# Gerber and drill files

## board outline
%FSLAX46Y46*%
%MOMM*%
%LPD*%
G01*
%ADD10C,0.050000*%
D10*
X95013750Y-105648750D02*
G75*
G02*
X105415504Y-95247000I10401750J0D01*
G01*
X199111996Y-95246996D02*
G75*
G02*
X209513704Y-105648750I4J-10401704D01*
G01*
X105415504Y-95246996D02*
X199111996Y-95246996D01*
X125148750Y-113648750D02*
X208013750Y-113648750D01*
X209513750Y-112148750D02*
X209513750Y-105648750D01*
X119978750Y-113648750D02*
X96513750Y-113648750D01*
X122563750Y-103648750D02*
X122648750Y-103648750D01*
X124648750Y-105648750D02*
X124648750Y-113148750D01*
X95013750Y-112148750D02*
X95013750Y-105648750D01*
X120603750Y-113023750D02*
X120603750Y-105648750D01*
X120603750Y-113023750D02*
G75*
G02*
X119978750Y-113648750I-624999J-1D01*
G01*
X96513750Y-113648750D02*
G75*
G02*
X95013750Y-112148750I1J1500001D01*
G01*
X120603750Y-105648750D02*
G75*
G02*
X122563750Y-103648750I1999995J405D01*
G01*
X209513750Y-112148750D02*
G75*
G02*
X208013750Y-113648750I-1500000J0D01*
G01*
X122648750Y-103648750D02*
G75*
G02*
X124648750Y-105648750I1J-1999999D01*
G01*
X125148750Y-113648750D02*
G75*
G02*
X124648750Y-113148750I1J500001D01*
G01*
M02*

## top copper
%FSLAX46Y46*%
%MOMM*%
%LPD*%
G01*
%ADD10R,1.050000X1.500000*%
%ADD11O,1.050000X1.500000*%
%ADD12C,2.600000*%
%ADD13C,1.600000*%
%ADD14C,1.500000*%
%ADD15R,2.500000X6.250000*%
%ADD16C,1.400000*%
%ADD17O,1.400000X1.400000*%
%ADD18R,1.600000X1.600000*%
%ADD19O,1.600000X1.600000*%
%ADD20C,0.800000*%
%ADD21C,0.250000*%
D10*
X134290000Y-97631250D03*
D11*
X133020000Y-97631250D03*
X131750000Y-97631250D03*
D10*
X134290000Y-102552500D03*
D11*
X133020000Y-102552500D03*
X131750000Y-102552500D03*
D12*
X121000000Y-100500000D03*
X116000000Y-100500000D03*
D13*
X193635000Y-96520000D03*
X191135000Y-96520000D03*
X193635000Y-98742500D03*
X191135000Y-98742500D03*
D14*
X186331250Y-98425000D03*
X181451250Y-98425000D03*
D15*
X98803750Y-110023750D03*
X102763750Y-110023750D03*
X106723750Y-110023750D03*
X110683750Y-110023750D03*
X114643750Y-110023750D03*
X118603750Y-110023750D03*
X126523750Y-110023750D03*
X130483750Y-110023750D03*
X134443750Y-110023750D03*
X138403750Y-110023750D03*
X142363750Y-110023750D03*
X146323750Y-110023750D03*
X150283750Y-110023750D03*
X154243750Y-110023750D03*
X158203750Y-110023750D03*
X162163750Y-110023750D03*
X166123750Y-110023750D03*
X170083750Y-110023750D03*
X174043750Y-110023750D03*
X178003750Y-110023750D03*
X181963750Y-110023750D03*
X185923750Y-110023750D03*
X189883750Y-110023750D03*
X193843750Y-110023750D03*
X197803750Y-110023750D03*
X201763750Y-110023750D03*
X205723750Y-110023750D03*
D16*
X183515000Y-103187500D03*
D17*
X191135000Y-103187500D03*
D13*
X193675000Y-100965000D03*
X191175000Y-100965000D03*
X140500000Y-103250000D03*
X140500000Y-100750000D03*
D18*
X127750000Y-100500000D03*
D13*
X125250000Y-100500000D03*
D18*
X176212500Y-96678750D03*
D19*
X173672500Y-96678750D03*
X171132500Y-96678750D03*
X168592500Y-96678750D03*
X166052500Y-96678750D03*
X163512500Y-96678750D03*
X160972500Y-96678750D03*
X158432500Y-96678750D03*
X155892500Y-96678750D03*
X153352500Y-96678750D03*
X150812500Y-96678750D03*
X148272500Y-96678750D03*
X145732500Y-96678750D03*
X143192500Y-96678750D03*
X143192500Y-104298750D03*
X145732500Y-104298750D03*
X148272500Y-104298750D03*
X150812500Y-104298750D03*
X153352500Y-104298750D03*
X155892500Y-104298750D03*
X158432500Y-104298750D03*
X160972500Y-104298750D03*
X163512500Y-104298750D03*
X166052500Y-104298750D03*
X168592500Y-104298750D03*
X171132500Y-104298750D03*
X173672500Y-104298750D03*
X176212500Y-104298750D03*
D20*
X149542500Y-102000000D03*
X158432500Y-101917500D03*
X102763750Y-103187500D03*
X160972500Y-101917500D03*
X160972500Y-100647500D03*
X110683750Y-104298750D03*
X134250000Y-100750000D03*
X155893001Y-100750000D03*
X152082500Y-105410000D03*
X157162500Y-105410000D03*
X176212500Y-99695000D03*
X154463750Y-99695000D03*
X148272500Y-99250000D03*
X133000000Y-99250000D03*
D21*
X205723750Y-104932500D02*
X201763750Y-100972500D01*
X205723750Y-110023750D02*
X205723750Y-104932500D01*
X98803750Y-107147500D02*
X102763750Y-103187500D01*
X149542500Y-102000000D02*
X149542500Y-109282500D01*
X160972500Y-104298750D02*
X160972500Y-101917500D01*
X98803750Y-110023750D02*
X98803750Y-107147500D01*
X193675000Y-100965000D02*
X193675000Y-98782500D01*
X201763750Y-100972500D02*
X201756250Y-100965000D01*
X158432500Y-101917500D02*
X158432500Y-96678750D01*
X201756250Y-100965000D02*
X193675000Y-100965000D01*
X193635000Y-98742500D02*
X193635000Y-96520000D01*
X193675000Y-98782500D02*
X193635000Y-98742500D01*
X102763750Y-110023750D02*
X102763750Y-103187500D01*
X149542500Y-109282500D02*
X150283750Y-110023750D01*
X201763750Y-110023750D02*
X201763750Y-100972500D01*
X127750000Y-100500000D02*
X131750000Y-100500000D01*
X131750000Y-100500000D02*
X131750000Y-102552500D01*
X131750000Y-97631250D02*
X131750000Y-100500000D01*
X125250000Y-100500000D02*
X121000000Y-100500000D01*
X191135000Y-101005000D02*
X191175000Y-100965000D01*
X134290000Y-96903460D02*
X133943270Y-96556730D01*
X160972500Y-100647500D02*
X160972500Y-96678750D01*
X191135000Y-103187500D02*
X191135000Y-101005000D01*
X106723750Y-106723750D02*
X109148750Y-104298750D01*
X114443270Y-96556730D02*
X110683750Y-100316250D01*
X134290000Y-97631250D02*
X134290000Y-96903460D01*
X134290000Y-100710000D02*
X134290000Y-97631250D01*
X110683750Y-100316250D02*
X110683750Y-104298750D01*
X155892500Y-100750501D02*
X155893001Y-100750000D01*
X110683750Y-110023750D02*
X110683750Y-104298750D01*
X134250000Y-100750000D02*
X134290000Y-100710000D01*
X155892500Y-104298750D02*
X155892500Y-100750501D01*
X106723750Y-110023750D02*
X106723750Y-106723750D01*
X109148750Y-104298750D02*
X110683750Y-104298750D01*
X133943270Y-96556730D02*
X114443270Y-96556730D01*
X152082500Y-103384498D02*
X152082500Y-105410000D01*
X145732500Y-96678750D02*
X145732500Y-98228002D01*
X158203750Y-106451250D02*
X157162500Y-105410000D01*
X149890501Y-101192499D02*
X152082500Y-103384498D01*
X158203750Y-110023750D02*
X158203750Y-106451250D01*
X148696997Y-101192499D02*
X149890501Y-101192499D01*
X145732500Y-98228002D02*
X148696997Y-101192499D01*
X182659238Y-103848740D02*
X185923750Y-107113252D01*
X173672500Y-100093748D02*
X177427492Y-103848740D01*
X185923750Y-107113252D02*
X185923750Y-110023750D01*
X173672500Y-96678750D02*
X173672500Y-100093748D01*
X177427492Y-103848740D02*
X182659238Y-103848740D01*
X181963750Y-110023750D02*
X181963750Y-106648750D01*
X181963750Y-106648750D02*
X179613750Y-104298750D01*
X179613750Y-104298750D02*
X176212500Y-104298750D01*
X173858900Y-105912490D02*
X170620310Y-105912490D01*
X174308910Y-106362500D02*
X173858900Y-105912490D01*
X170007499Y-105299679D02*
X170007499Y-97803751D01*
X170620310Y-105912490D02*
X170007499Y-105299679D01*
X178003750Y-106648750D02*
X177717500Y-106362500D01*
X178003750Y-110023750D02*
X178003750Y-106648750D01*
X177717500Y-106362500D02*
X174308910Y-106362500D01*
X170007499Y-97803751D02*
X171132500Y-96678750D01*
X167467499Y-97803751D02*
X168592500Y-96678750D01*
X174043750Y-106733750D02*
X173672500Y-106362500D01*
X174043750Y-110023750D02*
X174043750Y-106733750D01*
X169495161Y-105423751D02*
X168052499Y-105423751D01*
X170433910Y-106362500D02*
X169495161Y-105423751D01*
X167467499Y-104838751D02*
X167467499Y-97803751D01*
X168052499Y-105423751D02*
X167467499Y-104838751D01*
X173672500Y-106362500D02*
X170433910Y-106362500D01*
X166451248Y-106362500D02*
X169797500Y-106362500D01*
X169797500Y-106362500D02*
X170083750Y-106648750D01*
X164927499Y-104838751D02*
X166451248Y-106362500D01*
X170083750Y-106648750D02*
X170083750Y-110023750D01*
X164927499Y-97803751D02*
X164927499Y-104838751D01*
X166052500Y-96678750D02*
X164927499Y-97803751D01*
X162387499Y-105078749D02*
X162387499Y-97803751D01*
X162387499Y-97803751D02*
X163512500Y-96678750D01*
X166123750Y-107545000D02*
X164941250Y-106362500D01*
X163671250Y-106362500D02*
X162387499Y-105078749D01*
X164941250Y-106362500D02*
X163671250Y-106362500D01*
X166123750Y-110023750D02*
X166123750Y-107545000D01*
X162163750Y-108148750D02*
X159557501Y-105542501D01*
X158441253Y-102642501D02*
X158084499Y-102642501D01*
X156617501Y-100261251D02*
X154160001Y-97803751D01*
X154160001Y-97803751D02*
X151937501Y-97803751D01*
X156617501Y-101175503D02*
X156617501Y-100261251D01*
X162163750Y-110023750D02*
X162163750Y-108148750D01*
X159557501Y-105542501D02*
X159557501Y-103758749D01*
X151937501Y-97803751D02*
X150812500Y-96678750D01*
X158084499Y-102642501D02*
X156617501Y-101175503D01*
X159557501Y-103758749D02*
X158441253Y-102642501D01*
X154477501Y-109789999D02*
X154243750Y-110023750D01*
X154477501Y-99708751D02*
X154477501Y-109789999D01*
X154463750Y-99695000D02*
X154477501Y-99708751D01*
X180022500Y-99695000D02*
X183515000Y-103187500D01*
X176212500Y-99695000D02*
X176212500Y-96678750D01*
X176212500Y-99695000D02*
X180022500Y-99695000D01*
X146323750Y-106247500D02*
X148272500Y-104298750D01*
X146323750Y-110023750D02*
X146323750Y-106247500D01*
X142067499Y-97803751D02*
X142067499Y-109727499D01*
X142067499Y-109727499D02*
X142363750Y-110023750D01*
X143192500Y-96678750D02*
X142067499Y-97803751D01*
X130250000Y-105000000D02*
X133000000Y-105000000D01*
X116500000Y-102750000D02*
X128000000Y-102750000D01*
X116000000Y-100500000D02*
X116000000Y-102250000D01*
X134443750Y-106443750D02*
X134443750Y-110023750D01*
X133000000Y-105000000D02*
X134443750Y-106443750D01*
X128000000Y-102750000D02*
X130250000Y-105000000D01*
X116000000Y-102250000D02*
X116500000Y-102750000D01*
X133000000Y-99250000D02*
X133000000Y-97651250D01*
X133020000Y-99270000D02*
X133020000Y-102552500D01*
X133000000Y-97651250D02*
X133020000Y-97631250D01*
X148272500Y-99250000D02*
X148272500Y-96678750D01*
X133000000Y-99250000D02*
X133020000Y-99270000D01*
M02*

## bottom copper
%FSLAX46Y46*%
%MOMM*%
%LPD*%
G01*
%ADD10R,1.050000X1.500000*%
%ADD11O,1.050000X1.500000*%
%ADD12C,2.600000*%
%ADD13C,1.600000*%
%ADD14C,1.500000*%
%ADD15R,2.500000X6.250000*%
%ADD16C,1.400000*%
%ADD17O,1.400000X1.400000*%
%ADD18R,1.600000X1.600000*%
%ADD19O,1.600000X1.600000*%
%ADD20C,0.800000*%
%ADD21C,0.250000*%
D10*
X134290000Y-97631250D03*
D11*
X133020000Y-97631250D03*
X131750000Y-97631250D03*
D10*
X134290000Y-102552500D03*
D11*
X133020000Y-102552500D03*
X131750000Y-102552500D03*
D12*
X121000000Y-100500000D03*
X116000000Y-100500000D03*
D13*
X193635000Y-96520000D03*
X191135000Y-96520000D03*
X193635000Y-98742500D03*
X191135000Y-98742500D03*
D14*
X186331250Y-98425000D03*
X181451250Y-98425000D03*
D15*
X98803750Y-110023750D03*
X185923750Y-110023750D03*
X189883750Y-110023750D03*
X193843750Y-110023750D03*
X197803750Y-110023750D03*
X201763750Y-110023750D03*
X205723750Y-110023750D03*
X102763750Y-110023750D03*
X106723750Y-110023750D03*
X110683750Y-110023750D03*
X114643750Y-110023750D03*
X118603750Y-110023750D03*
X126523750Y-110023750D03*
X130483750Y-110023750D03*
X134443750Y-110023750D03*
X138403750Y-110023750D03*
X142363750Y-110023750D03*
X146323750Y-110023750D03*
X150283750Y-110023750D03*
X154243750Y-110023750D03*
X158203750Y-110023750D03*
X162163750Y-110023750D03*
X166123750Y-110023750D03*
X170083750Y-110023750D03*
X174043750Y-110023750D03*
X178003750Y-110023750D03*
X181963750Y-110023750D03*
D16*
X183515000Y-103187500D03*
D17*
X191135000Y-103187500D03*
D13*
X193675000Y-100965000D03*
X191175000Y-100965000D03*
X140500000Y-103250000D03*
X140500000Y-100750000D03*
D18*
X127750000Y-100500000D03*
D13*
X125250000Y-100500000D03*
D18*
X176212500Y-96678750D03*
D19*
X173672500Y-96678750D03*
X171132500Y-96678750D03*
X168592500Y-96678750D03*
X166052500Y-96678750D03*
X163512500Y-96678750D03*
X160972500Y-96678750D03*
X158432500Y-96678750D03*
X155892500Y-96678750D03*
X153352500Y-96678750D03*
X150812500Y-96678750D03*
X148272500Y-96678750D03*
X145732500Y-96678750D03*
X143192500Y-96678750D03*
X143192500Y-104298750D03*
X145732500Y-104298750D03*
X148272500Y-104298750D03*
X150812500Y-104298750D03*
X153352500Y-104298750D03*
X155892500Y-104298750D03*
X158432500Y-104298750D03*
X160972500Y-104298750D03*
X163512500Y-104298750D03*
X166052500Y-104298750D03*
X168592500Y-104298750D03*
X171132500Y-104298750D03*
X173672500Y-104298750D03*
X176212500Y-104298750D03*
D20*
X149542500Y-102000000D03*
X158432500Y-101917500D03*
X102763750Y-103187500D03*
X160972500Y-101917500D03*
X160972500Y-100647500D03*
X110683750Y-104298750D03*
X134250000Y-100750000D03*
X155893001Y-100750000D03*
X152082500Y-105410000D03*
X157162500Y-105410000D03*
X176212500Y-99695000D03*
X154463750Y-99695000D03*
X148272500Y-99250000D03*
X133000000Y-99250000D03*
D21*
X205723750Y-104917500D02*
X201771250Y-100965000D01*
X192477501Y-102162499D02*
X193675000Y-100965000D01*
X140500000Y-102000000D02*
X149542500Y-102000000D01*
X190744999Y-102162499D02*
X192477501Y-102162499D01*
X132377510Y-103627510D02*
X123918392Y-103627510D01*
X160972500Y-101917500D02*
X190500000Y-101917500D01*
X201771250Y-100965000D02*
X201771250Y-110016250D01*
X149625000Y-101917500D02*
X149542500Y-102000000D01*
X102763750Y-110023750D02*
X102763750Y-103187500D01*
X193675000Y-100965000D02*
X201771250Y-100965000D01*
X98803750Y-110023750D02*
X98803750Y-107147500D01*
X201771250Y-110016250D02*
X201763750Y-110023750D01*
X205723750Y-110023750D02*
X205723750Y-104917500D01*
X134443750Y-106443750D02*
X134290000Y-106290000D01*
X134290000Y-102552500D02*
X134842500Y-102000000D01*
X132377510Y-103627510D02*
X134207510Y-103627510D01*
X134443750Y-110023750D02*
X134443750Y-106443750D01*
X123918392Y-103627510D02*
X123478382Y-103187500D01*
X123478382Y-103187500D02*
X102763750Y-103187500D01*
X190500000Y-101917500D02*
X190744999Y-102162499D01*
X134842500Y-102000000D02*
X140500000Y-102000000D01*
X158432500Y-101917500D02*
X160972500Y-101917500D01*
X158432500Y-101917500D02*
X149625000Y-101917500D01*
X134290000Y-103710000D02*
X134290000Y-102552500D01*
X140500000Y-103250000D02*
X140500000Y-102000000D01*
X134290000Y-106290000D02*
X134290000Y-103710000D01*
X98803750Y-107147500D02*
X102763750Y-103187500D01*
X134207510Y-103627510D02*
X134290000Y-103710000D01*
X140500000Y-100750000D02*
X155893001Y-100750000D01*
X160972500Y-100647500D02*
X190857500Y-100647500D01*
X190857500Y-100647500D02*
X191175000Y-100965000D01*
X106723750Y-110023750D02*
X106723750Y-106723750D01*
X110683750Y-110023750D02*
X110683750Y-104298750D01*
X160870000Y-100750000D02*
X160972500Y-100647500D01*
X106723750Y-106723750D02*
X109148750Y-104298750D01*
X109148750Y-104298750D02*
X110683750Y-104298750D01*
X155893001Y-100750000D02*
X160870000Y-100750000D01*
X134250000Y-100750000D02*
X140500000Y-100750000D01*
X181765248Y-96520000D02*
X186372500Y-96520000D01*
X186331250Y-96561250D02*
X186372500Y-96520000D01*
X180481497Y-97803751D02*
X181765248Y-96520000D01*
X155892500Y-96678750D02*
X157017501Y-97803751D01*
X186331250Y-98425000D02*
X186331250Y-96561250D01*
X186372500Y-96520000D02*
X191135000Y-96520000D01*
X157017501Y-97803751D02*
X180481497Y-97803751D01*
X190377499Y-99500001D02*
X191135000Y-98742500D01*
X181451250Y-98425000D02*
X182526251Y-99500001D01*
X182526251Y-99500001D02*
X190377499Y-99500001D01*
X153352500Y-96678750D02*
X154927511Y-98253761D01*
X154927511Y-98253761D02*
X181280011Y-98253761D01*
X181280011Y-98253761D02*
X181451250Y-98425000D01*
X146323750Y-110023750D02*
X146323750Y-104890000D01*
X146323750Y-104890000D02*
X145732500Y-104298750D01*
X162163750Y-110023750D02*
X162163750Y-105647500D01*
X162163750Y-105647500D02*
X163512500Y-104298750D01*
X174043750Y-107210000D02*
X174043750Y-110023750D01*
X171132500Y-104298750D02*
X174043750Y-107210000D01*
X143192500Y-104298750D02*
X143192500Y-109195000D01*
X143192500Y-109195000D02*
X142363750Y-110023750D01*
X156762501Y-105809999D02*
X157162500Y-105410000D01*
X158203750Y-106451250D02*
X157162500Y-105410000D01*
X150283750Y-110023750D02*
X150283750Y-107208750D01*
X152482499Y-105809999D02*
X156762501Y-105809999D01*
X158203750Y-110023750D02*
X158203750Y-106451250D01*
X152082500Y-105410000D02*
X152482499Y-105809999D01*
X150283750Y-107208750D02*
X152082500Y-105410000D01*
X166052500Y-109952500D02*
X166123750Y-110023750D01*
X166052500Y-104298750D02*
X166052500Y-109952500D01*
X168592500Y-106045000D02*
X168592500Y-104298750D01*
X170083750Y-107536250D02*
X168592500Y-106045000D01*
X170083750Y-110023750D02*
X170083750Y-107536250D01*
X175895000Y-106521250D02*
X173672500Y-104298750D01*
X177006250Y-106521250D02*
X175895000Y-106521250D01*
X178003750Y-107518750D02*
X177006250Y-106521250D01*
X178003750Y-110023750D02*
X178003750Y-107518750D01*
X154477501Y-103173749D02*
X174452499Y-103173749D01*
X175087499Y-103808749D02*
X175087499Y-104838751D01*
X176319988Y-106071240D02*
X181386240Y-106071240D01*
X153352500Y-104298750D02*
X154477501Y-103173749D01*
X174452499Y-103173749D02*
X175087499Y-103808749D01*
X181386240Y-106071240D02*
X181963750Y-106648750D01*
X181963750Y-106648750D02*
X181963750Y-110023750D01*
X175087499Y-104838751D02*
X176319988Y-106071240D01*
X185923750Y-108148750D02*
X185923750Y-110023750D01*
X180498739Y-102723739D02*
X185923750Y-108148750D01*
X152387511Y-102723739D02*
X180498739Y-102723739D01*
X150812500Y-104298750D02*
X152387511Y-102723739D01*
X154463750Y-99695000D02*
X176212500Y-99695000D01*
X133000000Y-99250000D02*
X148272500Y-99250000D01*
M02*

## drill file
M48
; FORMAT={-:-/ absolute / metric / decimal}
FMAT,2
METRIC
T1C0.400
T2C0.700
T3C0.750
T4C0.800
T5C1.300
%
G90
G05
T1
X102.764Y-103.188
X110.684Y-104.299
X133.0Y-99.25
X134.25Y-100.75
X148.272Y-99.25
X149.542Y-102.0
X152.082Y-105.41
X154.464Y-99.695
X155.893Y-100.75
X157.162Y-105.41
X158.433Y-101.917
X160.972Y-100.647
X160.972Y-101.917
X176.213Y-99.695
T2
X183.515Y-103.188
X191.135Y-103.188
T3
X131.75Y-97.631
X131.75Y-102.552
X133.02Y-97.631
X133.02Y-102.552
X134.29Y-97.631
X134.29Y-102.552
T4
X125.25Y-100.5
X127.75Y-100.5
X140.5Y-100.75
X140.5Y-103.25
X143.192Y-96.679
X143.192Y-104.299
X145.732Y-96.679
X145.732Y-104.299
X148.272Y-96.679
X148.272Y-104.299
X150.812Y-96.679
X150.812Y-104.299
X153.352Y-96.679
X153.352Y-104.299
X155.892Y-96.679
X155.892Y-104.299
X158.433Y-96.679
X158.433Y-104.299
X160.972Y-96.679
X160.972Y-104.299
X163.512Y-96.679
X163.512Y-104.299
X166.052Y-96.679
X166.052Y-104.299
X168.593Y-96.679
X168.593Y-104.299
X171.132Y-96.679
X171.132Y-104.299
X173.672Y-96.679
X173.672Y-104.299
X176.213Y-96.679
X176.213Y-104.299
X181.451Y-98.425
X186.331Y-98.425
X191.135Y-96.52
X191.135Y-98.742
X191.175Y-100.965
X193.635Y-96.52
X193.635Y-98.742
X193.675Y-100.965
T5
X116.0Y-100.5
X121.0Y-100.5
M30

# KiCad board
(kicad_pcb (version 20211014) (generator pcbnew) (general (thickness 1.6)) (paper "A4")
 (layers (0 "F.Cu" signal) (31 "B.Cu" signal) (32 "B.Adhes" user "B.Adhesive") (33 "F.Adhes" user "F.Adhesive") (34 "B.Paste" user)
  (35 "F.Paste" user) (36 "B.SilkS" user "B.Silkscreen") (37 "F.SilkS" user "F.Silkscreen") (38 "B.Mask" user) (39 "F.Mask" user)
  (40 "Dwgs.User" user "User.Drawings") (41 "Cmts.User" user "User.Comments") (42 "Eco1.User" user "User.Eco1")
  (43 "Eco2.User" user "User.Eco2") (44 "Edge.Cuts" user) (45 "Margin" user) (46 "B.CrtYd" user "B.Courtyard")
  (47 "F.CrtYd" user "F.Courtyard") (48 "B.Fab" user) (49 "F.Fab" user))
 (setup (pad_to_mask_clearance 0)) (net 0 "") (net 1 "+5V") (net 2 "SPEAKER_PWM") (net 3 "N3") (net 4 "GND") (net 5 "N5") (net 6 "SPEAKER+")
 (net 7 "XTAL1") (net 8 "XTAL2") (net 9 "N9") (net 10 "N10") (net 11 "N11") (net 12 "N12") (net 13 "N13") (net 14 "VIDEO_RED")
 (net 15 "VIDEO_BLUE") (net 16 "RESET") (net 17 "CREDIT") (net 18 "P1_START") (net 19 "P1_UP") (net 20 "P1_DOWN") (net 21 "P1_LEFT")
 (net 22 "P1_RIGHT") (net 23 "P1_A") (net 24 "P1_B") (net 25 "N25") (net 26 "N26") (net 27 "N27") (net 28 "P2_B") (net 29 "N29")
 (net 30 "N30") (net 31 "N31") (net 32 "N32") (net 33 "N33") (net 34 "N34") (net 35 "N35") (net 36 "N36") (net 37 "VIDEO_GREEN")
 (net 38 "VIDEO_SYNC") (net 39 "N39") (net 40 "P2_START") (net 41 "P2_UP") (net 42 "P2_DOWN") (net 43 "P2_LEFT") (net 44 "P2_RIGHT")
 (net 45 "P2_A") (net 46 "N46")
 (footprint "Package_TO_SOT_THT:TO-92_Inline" (layer "F.Cu") (at 134.29 97.63125 180)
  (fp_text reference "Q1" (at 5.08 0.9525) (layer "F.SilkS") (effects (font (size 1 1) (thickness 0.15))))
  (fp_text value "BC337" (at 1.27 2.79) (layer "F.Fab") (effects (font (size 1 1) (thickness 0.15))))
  (pad "1" thru_hole rect locked (at 0 0 180) (size 1.05 1.5) (drill 0.75) (layers *.Cu *.Mask) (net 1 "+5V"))
  (pad "2" thru_hole oval locked (at 1.27 0 180) (size 1.05 1.5) (drill 0.75) (layers *.Cu *.Mask) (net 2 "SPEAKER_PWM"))
  (pad "3" thru_hole oval locked (at 2.54 0 180) (size 1.05 1.5) (drill 0.75) (layers *.Cu *.Mask) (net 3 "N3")))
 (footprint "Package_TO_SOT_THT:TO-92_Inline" (layer "F.Cu") (at 134.29 102.5525 180)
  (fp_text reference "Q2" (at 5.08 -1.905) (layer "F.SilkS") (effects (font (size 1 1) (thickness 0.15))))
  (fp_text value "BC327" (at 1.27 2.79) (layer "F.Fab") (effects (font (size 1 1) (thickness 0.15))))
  (pad "1" thru_hole rect locked (at 0 0 180) (size 1.05 1.5) (drill 0.75) (layers *.Cu *.Mask) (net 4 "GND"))
  (pad "2" thru_hole oval locked (at 1.27 0 180) (size 1.05 1.5) (drill 0.75) (layers *.Cu *.Mask) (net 2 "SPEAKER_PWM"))
  (pad "3" thru_hole oval locked (at 2.54 0 180) (size 1.05 1.5) (drill 0.75) (layers *.Cu *.Mask) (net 3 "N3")))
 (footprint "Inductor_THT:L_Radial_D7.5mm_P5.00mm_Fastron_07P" (layer "F.Cu") (at 121 100.5 180)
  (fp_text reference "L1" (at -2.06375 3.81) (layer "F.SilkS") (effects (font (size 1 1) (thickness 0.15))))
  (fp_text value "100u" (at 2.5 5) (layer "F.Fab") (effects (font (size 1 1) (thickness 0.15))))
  (pad "1" thru_hole circle locked (at 0 0 180) (size 2.6 2.6) (drill 1.3) (layers *.Cu *.Mask) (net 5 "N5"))
  (pad "2" thru_hole circle locked (at 5 0 180) (size 2.6 2.6) (drill 1.3) (layers *.Cu *.Mask) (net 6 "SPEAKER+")))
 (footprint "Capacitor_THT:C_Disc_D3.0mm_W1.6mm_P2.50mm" (layer "F.Cu") (at 193.635 96.52 180)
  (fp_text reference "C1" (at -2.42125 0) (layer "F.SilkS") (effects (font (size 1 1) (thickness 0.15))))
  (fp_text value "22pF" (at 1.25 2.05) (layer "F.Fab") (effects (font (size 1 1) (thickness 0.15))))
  (pad "1" thru_hole circle locked (at 0 0 180) (size 1.6 1.6) (drill 0.8) (layers *.Cu *.Mask) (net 4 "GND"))
  (pad "2" thru_hole circle locked (at 2.5 0 180) (size 1.6 1.6) (drill 0.8) (layers *.Cu *.Mask) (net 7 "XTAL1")))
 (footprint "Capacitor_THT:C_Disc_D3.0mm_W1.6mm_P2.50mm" (layer "F.Cu") (at 193.635 98.7425 180)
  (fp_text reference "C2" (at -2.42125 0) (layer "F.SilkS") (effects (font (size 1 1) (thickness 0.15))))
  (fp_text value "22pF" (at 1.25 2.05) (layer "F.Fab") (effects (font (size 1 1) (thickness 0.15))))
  (pad "1" thru_hole circle locked (at 0 0 180) (size 1.6 1.6) (drill 0.8) (layers *.Cu *.Mask) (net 4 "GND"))
  (pad "2" thru_hole circle locked (at 2.5 0 180) (size 1.6 1.6) (drill 0.8) (layers *.Cu *.Mask) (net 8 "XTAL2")))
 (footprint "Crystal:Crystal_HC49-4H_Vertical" (layer "F.Cu") (at 186.33125 98.425 180)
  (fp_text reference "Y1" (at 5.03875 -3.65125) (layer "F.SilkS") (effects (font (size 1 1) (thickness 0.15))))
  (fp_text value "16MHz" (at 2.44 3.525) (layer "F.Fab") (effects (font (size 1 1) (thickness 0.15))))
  (pad "1" thru_hole circle locked (at 0 0 180) (size 1.5 1.5) (drill 0.8) (layers *.Cu *.Mask) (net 7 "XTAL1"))
  (pad "2" thru_hole circle locked (at 4.88 0 180) (size 1.5 1.5) (drill 0.8) (layers *.Cu *.Mask) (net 8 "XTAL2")))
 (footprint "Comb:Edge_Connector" (layer "F.Cu") (at 152.26375 105.64875)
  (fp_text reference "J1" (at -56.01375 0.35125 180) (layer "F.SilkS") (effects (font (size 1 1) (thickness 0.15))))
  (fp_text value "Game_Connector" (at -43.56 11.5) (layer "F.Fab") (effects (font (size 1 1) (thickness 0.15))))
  (fp_line (start -27.115 8) (end 55.75 8) (layer "Edge.Cuts") (width 0.05))
  (fp_line (start 57.25 6.5) (end 57.25 0) (layer "Edge.Cuts") (width 0.05))
  (fp_line (start -32.285 8) (end -55.75 8) (layer "Edge.Cuts") (width 0.05))
  (fp_line (start -29.7 -2) (end -29.615 -2) (layer "Edge.Cuts") (width 0.05))
  (fp_line (start -27.615 0) (end -27.615 7.5) (layer "Edge.Cuts") (width 0.05))
  (fp_line (start -57.25 6.5) (end -57.25 0) (layer "Edge.Cuts") (width 0.05))
  (fp_line (start -31.66 7.375) (end -31.66 0) (layer "Edge.Cuts") (width 0.05))
  (fp_arc (start -31.66 7.375) (mid -31.843058 7.816942) (end -32.285 8) (layer "Edge.Cuts") (width 0.05))
  (fp_arc (start -55.75 8) (mid -56.81066 7.56066) (end -57.25 6.5) (layer "Edge.Cuts") (width 0.05))
  (fp_arc (start -31.66 0) (mid -31.088427 -1.400259) (end -29.7 -2) (layer "Edge.Cuts") (width 0.05))
  (fp_arc (start 57.25 6.5) (mid 56.81066 7.56066) (end 55.75 8) (layer "Edge.Cuts") (width 0.05))
  (fp_arc (start -29.615 -2) (mid -28.200786 -1.414214) (end -27.615 0) (layer "Edge.Cuts") (width 0.05))
  (fp_arc (start -27.115 8) (mid -27.468553 7.853553) (end -27.615 7.5) (layer "Edge.Cuts") (width 0.05))
  (pad "1" smd rect (at -53.46 4.375) (size 2.5 6.25) (layers "F.Cu" "F.Paste" "F.Mask") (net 4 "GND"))
  (pad "2" smd rect (at -49.5 4.375) (size 2.5 6.25) (layers "F.Cu" "F.Paste" "F.Mask") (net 4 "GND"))
  (pad "3" smd rect (at -45.54 4.375) (size 2.5 6.25) (layers "F.Cu" "F.Paste" "F.Mask") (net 1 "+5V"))
  (pad "4" smd rect (at -41.58 4.375) (size 2.5 6.25) (layers "F.Cu" "F.Paste" "F.Mask") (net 1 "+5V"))
  (pad "5" smd rect (at -37.62 4.375) (size 2.5 6.25) (layers "F.Cu" "F.Paste" "F.Mask") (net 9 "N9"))
  (pad "6" smd rect (at -33.66 4.375) (size 2.5 6.25) (layers "F.Cu" "F.Paste" "F.Mask") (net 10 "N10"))
  (pad "8" smd rect (at -25.74 4.375) (size 2.5 6.25) (layers "F.Cu" "F.Paste" "F.Mask") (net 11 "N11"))
  (pad "9" smd rect (at -21.78 4.375) (size 2.5 6.25) (layers "F.Cu" "F.Paste" "F.Mask") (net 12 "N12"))
  (pad "10" smd rect (at -17.82 4.375) (size 2.5 6.25) (layers "F.Cu" "F.Paste" "F.Mask") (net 6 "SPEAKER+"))
  (pad "11" smd rect (at -13.86 4.375) (size 2.5 6.25) (layers "F.Cu" "F.Paste" "F.Mask") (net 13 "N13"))
  (pad "12" smd rect (at -9.9 4.375) (size 2.5 6.25) (layers "F.Cu" "F.Paste" "F.Mask") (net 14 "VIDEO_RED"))
  (pad "13" smd rect (at -5.94 4.375) (size 2.5 6.25) (layers "F.Cu" "F.Paste" "F.Mask") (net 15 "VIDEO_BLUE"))
  (pad "14" smd rect (at -1.98 4.375) (size 2.5 6.25) (layers "F.Cu" "F.Paste" "F.Mask") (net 4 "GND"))
  (pad "15" smd rect (at 1.98 4.375) (size 2.5 6.25) (layers "F.Cu" "F.Paste" "F.Mask") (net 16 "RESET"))
  (pad "16" smd rect (at 5.94 4.375) (size 2.5 6.25) (layers "F.Cu" "F.Paste" "F.Mask") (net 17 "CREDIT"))
  (pad "17" smd rect (at 9.9 4.375) (size 2.5 6.25) (layers "F.Cu" "F.Paste" "F.Mask") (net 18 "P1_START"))
  (pad "18" smd rect (at 13.86 4.375) (size 2.5 6.25) (layers "F.Cu" "F.Paste" "F.Mask") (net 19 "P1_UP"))
  (pad "19" smd rect (at 17.82 4.375) (size 2.5 6.25) (layers "F.Cu" "F.Paste" "F.Mask") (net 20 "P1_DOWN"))
  (pad "20" smd rect (at 21.78 4.375) (size 2.5 6.25) (layers "F.Cu" "F.Paste" "F.Mask") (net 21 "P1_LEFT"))
  (pad "21" smd rect (at 25.74 4.375) (size 2.5 6.25) (layers "F.Cu" "F.Paste" "F.Mask") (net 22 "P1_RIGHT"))
  (pad "22" smd rect (at 29.7 4.375) (size 2.5 6.25) (layers "F.Cu" "F.Paste" "F.Mask") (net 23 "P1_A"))
  (pad "23" smd rect (at 33.66 4.375) (size 2.5 6.25) (layers "F.Cu" "F.Paste" "F.Mask") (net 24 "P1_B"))
  (pad "24" smd rect (at 37.62 4.375) (size 2.5 6.25) (layers "F.Cu" "F.Paste" "F.Mask") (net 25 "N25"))
  (pad "25" smd rect (at 41.58 4.375) (size 2.5 6.25) (layers "F.Cu" "F.Paste" "F.Mask") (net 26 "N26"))
  (pad "26" smd rect (at 45.54 4.375) (size 2.5 6.25) (layers "F.Cu" "F.Paste" "F.Mask") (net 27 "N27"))
  (pad "27" smd rect (at 49.5 4.375) (size 2.5 6.25) (layers "F.Cu" "F.Paste" "F.Mask") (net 4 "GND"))
  (pad "28" smd rect (at 53.46 4.375) (size 2.5 6.25) (layers "F.Cu" "F.Paste" "F.Mask") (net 4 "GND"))
  (pad "A" smd rect (at -53.46 4.375) (size 2.5 6.25) (layers "B.Cu" "B.Paste" "B.Mask") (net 4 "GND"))
  (pad "AA" smd rect (at 33.66 4.375) (size 2.5 6.25) (layers "B.Cu" "B.Paste" "B.Mask") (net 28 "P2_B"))
  (pad "AB" smd rect (at 37.62 4.375) (size 2.5 6.25) (layers "B.Cu" "B.Paste" "B.Mask") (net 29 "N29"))
  (pad "AC" smd rect (at 41.58 4.375) (size 2.5 6.25) (layers "B.Cu" "B.Paste" "B.Mask") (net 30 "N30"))
  (pad "AD" smd rect (at 45.54 4.375) (size 2.5 6.25) (layers "B.Cu" "B.Paste" "B.Mask") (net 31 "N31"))
  (pad "AE" smd rect (at 49.5 4.375) (size 2.5 6.25) (layers "B.Cu" "B.Paste" "B.Mask") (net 4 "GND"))
  (pad "AF" smd rect (at 53.46 4.375) (size 2.5 6.25) (layers "B.Cu" "B.Paste" "B.Mask") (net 4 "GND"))
  (pad "B" smd rect (at -49.5 4.375) (size 2.5 6.25) (layers "B.Cu" "B.Paste" "B.Mask") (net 4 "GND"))
  (pad "C" smd rect (at -45.54 4.375) (size 2.5 6.25) (layers "B.Cu" "B.Paste" "B.Mask") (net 1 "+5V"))
  (pad "D" smd rect (at -41.58 4.375) (size 2.5 6.25) (layers "B.Cu" "B.Paste" "B.Mask") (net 1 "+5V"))
  (pad "E" smd rect (at -37.62 4.375) (size 2.5 6.25) (layers "B.Cu" "B.Paste" "B.Mask") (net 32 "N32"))
  (pad "F" smd rect (at -33.66 4.375) (size 2.5 6.25) (layers "B.Cu" "B.Paste" "B.Mask") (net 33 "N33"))
  (pad "J" smd rect (at -25.74 4.375) (size 2.5 6.25) (layers "B.Cu" "B.Paste" "B.Mask") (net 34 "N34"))
  (pad "K" smd rect (at -21.78 4.375) (size 2.5 6.25) (layers "B.Cu" "B.Paste" "B.Mask") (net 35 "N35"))
  (pad "L" smd rect (at -17.82 4.375) (size 2.5 6.25) (layers "B.Cu" "B.Paste" "B.Mask") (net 4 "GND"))
  (pad "M" smd rect (at -13.86 4.375) (size 2.5 6.25) (layers "B.Cu" "B.Paste" "B.Mask") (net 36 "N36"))
  (pad "N" smd rect (at -9.9 4.375) (size 2.5 6.25) (layers "B.Cu" "B.Paste" "B.Mask") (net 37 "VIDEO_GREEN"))
  (pad "P" smd rect (at -5.94 4.375) (size 2.5 6.25) (layers "B.Cu" "B.Paste" "B.Mask") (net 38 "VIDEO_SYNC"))
  (pad "R" smd rect (at -1.98 4.375) (size 2.5 6.25) (layers "B.Cu" "B.Paste" "B.Mask") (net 17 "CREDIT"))
  (pad "S" smd rect (at 1.98 4.375) (size 2.5 6.25) (layers "B.Cu" "B.Paste" "B.Mask") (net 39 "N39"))
  (pad "T" smd rect (at 5.94 4.375) (size 2.5 6.25) (layers "B.Cu" "B.Paste" "B.Mask") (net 17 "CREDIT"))
  (pad "U" smd rect (at 9.9 4.375) (size 2.5 6.25) (layers "B.Cu" "B.Paste" "B.Mask") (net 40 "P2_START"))
  (pad "V" smd rect (at 13.86 4.375) (size 2.5 6.25) (layers "B.Cu" "B.Paste" "B.Mask") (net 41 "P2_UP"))
  (pad "W" smd rect (at 17.82 4.375) (size 2.5 6.25) (layers "B.Cu" "B.Paste" "B.Mask") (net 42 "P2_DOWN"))
  (pad "X" smd rect (at 21.78 4.375) (size 2.5 6.25) (layers "B.Cu" "B.Paste" "B.Mask") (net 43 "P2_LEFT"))
  (pad "Y" smd rect (at 25.74 4.375) (size 2.5 6.25) (layers "B.Cu" "B.Paste" "B.Mask") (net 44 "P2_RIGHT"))
  (pad "Z" smd rect (at 29.7 4.375) (size 2.5 6.25) (layers "B.Cu" "B.Paste" "B.Mask") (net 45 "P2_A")))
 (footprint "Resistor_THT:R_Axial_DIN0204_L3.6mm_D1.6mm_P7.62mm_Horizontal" (layer "F.Cu") (at 183.515 103.1875)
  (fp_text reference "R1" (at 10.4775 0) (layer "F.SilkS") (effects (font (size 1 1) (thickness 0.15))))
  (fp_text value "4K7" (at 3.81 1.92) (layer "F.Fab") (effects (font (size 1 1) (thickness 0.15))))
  (pad "1" thru_hole circle locked (at 0 0) (size 1.4 1.4) (drill 0.7) (layers *.Cu *.Mask) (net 16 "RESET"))
  (pad "2" thru_hole oval locked (at 7.62 0) (size 1.4 1.4) (drill 0.7) (layers *.Cu *.Mask) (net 1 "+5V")))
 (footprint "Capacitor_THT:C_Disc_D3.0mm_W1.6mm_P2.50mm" (layer "F.Cu") (at 193.675 100.965 180)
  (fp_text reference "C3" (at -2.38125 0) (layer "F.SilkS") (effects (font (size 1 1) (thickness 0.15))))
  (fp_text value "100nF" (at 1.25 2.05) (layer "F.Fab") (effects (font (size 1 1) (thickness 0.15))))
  (pad "1" thru_hole circle locked (at 0 0 180) (size 1.6 1.6) (drill 0.8) (layers *.Cu *.Mask) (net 4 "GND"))
  (pad "2" thru_hole circle locked (at 2.5 0 180) (size 1.6 1.6) (drill 0.8) (layers *.Cu *.Mask) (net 1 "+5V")))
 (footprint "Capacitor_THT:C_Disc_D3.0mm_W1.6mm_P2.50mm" (layer "F.Cu") (at 140.5 103.25 90)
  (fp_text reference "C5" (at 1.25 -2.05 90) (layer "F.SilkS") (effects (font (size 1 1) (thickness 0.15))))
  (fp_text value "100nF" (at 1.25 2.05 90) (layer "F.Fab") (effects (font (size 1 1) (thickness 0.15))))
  (pad "1" thru_hole circle (at 0 0 90) (size 1.6 1.6) (drill 0.8) (layers *.Cu *.Mask) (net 4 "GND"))
  (pad "2" thru_hole circle (at 2.5 0 90) (size 1.6 1.6) (drill 0.8) (layers *.Cu *.Mask) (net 1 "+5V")))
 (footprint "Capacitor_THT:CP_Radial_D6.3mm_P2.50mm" (layer "F.Cu") (at 127.75 100.5 180)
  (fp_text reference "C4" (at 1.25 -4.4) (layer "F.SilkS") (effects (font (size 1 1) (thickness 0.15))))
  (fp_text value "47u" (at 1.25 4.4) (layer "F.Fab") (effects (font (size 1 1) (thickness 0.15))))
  (pad "1" thru_hole rect (at 0 0 180) (size 1.6 1.6) (drill 0.8) (layers *.Cu *.Mask) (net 3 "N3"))
  (pad "2" thru_hole circle (at 2.5 0 180) (size 1.6 1.6) (drill 0.8) (layers *.Cu *.Mask) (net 5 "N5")))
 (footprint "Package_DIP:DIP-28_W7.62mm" (layer "F.Cu") (at 176.2125 96.67875 -90)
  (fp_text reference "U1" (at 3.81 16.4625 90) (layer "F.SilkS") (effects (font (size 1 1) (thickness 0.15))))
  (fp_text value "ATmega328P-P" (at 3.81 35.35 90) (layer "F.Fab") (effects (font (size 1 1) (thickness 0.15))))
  (pad "1" thru_hole rect (at 0 0 270) (size 1.6 1.6) (drill 0.8) (layers *.Cu *.Mask) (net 16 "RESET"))
  (pad "2" thru_hole oval (at 0 2.54 270) (size 1.6 1.6) (drill 0.8) (layers *.Cu *.Mask) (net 24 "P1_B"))
  (pad "3" thru_hole oval (at 0 5.08 270) (size 1.6 1.6) (drill 0.8) (layers *.Cu *.Mask) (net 22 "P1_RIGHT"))
  (pad "4" thru_hole oval (at 0 7.62 270) (size 1.6 1.6) (drill 0.8) (layers *.Cu *.Mask) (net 21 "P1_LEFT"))
  (pad "5" thru_hole oval (at 0 10.16 270) (size 1.6 1.6) (drill 0.8) (layers *.Cu *.Mask) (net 20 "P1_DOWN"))
  (pad "6" thru_hole oval (at 0 12.7 270) (size 1.6 1.6) (drill 0.8) (layers *.Cu *.Mask) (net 19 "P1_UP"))
  (pad "7" thru_hole oval (at 0 15.24 270) (size 1.6 1.6) (drill 0.8) (layers *.Cu *.Mask) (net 1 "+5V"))
  (pad "8" thru_hole oval (at 0 17.78 270) (size 1.6 1.6) (drill 0.8) (layers *.Cu *.Mask) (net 4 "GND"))
  (pad "9" thru_hole oval (at 0 20.32 270) (size 1.6 1.6) (drill 0.8) (layers *.Cu *.Mask) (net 7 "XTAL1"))
  (pad "10" thru_hole oval (at 0 22.86 270) (size 1.6 1.6) (drill 0.8) (layers *.Cu *.Mask) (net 8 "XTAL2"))
  (pad "11" thru_hole oval (at 0 25.4 270) (size 1.6 1.6) (drill 0.8) (layers *.Cu *.Mask) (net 18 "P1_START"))
  (pad "12" thru_hole oval (at 0 27.94 270) (size 1.6 1.6) (drill 0.8) (layers *.Cu *.Mask) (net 2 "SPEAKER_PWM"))
  (pad "13" thru_hole oval (at 0 30.48 270) (size 1.6 1.6) (drill 0.8) (layers *.Cu *.Mask) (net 17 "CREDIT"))
  (pad "14" thru_hole oval (at 0 33.02 270) (size 1.6 1.6) (drill 0.8) (layers *.Cu *.Mask) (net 14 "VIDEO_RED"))
  (pad "15" thru_hole oval (at 7.62 33.02 270) (size 1.6 1.6) (drill 0.8) (layers *.Cu *.Mask) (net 37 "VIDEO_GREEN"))
  (pad "16" thru_hole oval (at 7.62 30.48 270) (size 1.6 1.6) (drill 0.8) (layers *.Cu *.Mask) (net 38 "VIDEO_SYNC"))
  (pad "17" thru_hole oval (at 7.62 27.94 270) (size 1.6 1.6) (drill 0.8) (layers *.Cu *.Mask) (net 15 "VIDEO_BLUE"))
  (pad "18" thru_hole oval (at 7.62 25.4 270) (size 1.6 1.6) (drill 0.8) (layers *.Cu *.Mask) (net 28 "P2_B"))
  (pad "19" thru_hole oval (at 7.62 22.86 270) (size 1.6 1.6) (drill 0.8) (layers *.Cu *.Mask) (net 45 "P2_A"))
  (pad "20" thru_hole oval (at 7.62 20.32 270) (size 1.6 1.6) (drill 0.8) (layers *.Cu *.Mask) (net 1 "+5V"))
  (pad "21" thru_hole oval (at 7.62 17.78 270) (size 1.6 1.6) (drill 0.8) (layers *.Cu *.Mask) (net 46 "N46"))
  (pad "22" thru_hole oval (at 7.62 15.24 270) (size 1.6 1.6) (drill 0.8) (layers *.Cu *.Mask) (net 4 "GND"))
  (pad "23" thru_hole oval (at 7.62 12.7 270) (size 1.6 1.6) (drill 0.8) (layers *.Cu *.Mask) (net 40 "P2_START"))
  (pad "24" thru_hole oval (at 7.62 10.16 270) (size 1.6 1.6) (drill 0.8) (layers *.Cu *.Mask) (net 41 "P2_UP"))
  (pad "25" thru_hole oval (at 7.62 7.62 270) (size 1.6 1.6) (drill 0.8) (layers *.Cu *.Mask) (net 42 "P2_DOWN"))
  (pad "26" thru_hole oval (at 7.62 5.08 270) (size 1.6 1.6) (drill 0.8) (layers *.Cu *.Mask) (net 43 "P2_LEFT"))
  (pad "27" thru_hole oval (at 7.62 2.54 270) (size 1.6 1.6) (drill 0.8) (layers *.Cu *.Mask) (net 44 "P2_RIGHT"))
  (pad "28" thru_hole oval (at 7.62 0 270) (size 1.6 1.6) (drill 0.8) (layers *.Cu *.Mask) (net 23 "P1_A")))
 (gr_arc (start 95.01375 105.64875) (mid 98.060353 98.293599) (end 105.415504 95.246996) (layer "Edge.Cuts") (width 0.05))
 (gr_arc (start 199.111996 95.246996) (mid 206.467147 98.293599) (end 209.51375 105.64875) (layer "Edge.Cuts") (width 0.05))
 (gr_line (start 105.415504 95.246996) (end 199.111996 95.246996) (layer "Edge.Cuts") (width 0.05))
 (segment (start 205.72375 104.9325) (end 201.76375 100.9725) (width 0.25) (layer "F.Cu") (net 4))
 (segment (start 205.72375 110.02375) (end 205.72375 104.9325) (width 0.25) (layer "F.Cu") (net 4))
 (segment (start 98.80375 107.1475) (end 102.76375 103.1875) (width 0.25) (layer "F.Cu") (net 4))
 (segment (start 149.5425 102) (end 149.5425 109.2825) (width 0.25) (layer "F.Cu") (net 4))
 (segment (start 160.9725 104.29875) (end 160.9725 101.9175) (width 0.25) (layer "F.Cu") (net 4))
 (segment (start 98.80375 110.02375) (end 98.80375 107.1475) (width 0.25) (layer "F.Cu") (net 4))
 (segment (start 193.675 100.965) (end 193.675 98.7825) (width 0.25) (layer "F.Cu") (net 4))
 (segment (start 201.76375 100.9725) (end 201.75625 100.965) (width 0.25) (layer "F.Cu") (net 4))
 (segment (start 158.4325 101.9175) (end 158.4325 96.67875) (width 0.25) (layer "F.Cu") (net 4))
 (segment (start 201.75625 100.965) (end 193.675 100.965) (width 0.25) (layer "F.Cu") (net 4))
 (segment (start 193.635 98.7425) (end 193.635 96.52) (width 0.25) (layer "F.Cu") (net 4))
 (segment (start 193.675 98.7825) (end 193.635 98.7425) (width 0.25) (layer "F.Cu") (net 4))
 (segment (start 102.76375 110.02375) (end 102.76375 103.1875) (width 0.25) (layer "F.Cu") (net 4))
 (segment (start 149.5425 109.2825) (end 150.28375 110.02375) (width 0.25) (layer "F.Cu") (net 4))
 (segment (start 201.76375 110.02375) (end 201.76375 100.9725) (width 0.25) (layer "F.Cu") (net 4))
 (via (at 149.5425 102) (size 0.8) (drill 0.4) (layers "F.Cu" "B.Cu") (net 4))
 (via (at 158.4325 101.9175) (size 0.8) (drill 0.4) (layers "F.Cu" "B.Cu") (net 4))
 (via (at 102.76375 103.1875) (size 0.8) (drill 0.4) (layers "F.Cu" "B.Cu") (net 4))
 (via (at 160.9725 101.9175) (size 0.8) (drill 0.4) (layers "F.Cu" "B.Cu") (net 4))
 (segment (start 205.72375 104.9175) (end 201.77125 100.965) (width 0.25) (layer "B.Cu") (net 4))
 (segment (start 192.477501 102.162499) (end 193.675 100.965) (width 0.25) (layer "B.Cu") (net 4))
 (segment (start 140.5 102) (end 149.5425 102) (width 0.25) (layer "B.Cu") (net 4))
 (segment (start 190.744999 102.162499) (end 192.477501 102.162499) (width 0.25) (layer "B.Cu") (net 4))
 (segment (start 132.37751 103.62751) (end 123.918392 103.62751) (width 0.25) (layer "B.Cu") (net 4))
 (segment (start 160.9725 101.9175) (end 190.5 101.9175) (width 0.25) (layer "B.Cu") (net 4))
 (segment (start 201.77125 100.965) (end 201.77125 110.01625) (width 0.25) (layer "B.Cu") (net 4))
 (segment (start 149.625 101.9175) (end 149.5425 102) (width 0.25) (layer "B.Cu") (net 4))
 (segment (start 102.76375 110.02375) (end 102.76375 103.1875) (width 0.25) (layer "B.Cu") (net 4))
 (segment (start 193.675 100.965) (end 201.77125 100.965) (width 0.25) (layer "B.Cu") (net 4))
 (segment (start 98.80375 110.02375) (end 98.80375 107.1475) (width 0.25) (layer "B.Cu") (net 4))
 (segment (start 201.77125 110.01625) (end 201.76375 110.02375) (width 0.25) (layer "B.Cu") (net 4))
 (segment (start 205.72375 110.02375) (end 205.72375 104.9175) (width 0.25) (layer "B.Cu") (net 4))
 (segment (start 134.44375 106.44375) (end 134.29 106.29) (width 0.25) (layer "B.Cu") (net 4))
 (segment (start 134.29 102.5525) (end 134.8425 102) (width 0.25) (layer "B.Cu") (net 4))
 (segment (start 132.37751 103.62751) (end 134.20751 103.62751) (width 0.25) (layer "B.Cu") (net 4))
 (segment (start 134.44375 110.02375) (end 134.44375 106.44375) (width 0.25) (layer "B.Cu") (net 4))
 (segment (start 123.918392 103.62751) (end 123.478382 103.1875) (width 0.25) (layer "B.Cu") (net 4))
 (segment (start 123.478382 103.1875) (end 102.76375 103.1875) (width 0.25) (layer "B.Cu") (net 4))
 (segment (start 190.5 101.9175) (end 190.744999 102.162499) (width 0.25) (layer "B.Cu") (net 4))
 (segment (start 134.8425 102) (end 140.5 102) (width 0.25) (layer "B.Cu") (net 4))
 (segment (start 158.4325 101.9175) (end 160.9725 101.9175) (width 0.25) (layer "B.Cu") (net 4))
 (segment (start 158.4325 101.9175) (end 149.625 101.9175) (width 0.25) (layer "B.Cu") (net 4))
 (segment (start 134.29 103.71) (end 134.29 102.5525) (width 0.25) (layer "B.Cu") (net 4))
 (segment (start 140.5 103.25) (end 140.5 102) (width 0.25) (layer "B.Cu") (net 4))
 (segment (start 134.29 106.29) (end 134.29 103.71) (width 0.25) (layer "B.Cu") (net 4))
 (segment (start 98.80375 107.1475) (end 102.76375 103.1875) (width 0.25) (layer "B.Cu") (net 4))
 (segment (start 134.20751 103.62751) (end 134.29 103.71) (width 0.25) (layer "B.Cu") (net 4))
 (segment (start 127.75 100.5) (end 131.75 100.5) (width 0.25) (layer "F.Cu") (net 3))
 (segment (start 131.75 100.5) (end 131.75 102.5525) (width 0.25) (layer "F.Cu") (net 3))
 (segment (start 131.75 97.63125) (end 131.75 100.5) (width 0.25) (layer "F.Cu") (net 3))
 (segment (start 125.25 100.5) (end 121 100.5) (width 0.25) (layer "F.Cu") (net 5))
 (segment (start 191.135 101.005) (end 191.175 100.965) (width 0.25) (layer "F.Cu") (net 1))
 (segment (start 134.29 96.90346) (end 133.94327 96.55673) (width 0.25) (layer "F.Cu") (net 1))
 (segment (start 160.9725 100.6475) (end 160.9725 96.67875) (width 0.25) (layer "F.Cu") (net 1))
 (segment (start 191.135 103.1875) (end 191.135 101.005) (width 0.25) (layer "F.Cu") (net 1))
 (segment (start 106.72375 106.72375) (end 109.14875 104.29875) (width 0.25) (layer "F.Cu") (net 1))
 (segment (start 114.44327 96.55673) (end 110.68375 100.31625) (width 0.25) (layer "F.Cu") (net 1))
 (segment (start 134.29 97.63125) (end 134.29 96.90346) (width 0.25) (layer "F.Cu") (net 1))
 (segment (start 134.29 100.71) (end 134.29 97.63125) (width 0.25) (layer "F.Cu") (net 1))
 (segment (start 110.68375 100.31625) (end 110.68375 104.29875) (width 0.25) (layer "F.Cu") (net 1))
 (segment (start 155.8925 100.750501) (end 155.893001 100.75) (width 0.25) (layer "F.Cu") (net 1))
 (segment (start 110.68375 110.02375) (end 110.68375 104.29875) (width 0.25) (layer "F.Cu") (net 1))
 (segment (start 134.25 100.75) (end 134.29 100.71) (width 0.25) (layer "F.Cu") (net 1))
 (segment (start 155.8925 104.29875) (end 155.8925 100.750501) (width 0.25) (layer "F.Cu") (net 1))
 (segment (start 106.72375 110.02375) (end 106.72375 106.72375) (width 0.25) (layer "F.Cu") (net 1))
 (segment (start 109.14875 104.29875) (end 110.68375 104.29875) (width 0.25) (layer "F.Cu") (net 1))
 (segment (start 133.94327 96.55673) (end 114.44327 96.55673) (width 0.25) (layer "F.Cu") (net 1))
 (via (at 160.9725 100.6475) (size 0.8) (drill 0.4) (layers "F.Cu" "B.Cu") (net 1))
 (via (at 110.68375 104.29875) (size 0.8) (drill 0.4) (layers "F.Cu" "B.Cu") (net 1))
 (via (at 134.25 100.75) (size 0.8) (drill 0.4) (layers "F.Cu" "B.Cu") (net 1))
 (via (at 155.893001 100.75) (size 0.8) (drill 0.4) (layers "F.Cu" "B.Cu") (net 1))
 (segment (start 140.5 100.75) (end 155.893001 100.75) (width 0.25) (layer "B.Cu") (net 1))
 (segment (start 160.9725 100.6475) (end 190.8575 100.6475) (width 0.25) (layer "B.Cu") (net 1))
 (segment (start 190.8575 100.6475) (end 191.175 100.965) (width 0.25) (layer "B.Cu") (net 1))
 (segment (start 106.72375 110.02375) (end 106.72375 106.72375) (width 0.25) (layer "B.Cu") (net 1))
 (segment (start 110.68375 110.02375) (end 110.68375 104.29875) (width 0.25) (layer "B.Cu") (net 1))
 (segment (start 160.87 100.75) (end 160.9725 100.6475) (width 0.25) (layer "B.Cu") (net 1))
 (segment (start 106.72375 106.72375) (end 109.14875 104.29875) (width 0.25) (layer "B.Cu") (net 1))
 (segment (start 109.14875 104.29875) (end 110.68375 104.29875) (width 0.25) (layer "B.Cu") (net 1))
 (segment (start 155.893001 100.75) (end 160.87 100.75) (width 0.25) (layer "B.Cu") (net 1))
 (segment (start 134.25 100.75) (end 140.5 100.75) (width 0.25) (layer "B.Cu") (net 1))
 (segment (start 181.765248 96.52) (end 186.3725 96.52) (width 0.25) (layer "B.Cu") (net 7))
 (segment (start 186.33125 96.56125) (end 186.3725 96.52) (width 0.25) (layer "B.Cu") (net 7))
 (segment (start 180.481497 97.803751) (end 181.765248 96.52) (width 0.25) (layer "B.Cu") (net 7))
 (segment (start 155.8925 96.67875) (end 157.017501 97.803751) (width 0.25) (layer "B.Cu") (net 7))
 (segment (start 186.33125 98.425) (end 186.33125 96.56125) (width 0.25) (layer "B.Cu") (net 7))
 (segment (start 186.3725 96.52) (end 191.135 96.52) (width 0.25) (layer "B.Cu") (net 7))
 (segment (start 157.017501 97.803751) (end 180.481497 97.803751) (width 0.25) (layer "B.Cu") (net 7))
 (segment (start 190.377499 99.500001) (end 191.135 98.7425) (width 0.25) (layer "B.Cu") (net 8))
 (segment (start 181.45125 98.425) (end 182.526251 99.500001) (width 0.25) (layer "B.Cu") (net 8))
 (segment (start 182.526251 99.500001) (end 190.377499 99.500001) (width 0.25) (layer "B.Cu") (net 8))
 (segment (start 153.3525 96.67875) (end 154.927511 98.253761) (width 0.25) (layer "B.Cu") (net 8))
 (segment (start 154.927511 98.253761) (end 181.280011 98.253761) (width 0.25) (layer "B.Cu") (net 8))
 (segment (start 181.280011 98.253761) (end 181.45125 98.425) (width 0.25) (layer "B.Cu") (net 8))
 (segment (start 146.32375 110.02375) (end 146.32375 104.89) (width 0.25) (layer "B.Cu") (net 38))
 (segment (start 146.32375 104.89) (end 145.7325 104.29875) (width 0.25) (layer "B.Cu") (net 38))
 (segment (start 162.16375 110.02375) (end 162.16375 105.6475) (width 0.25) (layer "B.Cu") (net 40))
 (segment (start 162.16375 105.6475) (end 163.5125 104.29875) (width 0.25) (layer "B.Cu") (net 40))
 (segment (start 174.04375 107.21) (end 174.04375 110.02375) (width 0.25) (layer "B.Cu") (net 43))
 (segment (start 171.1325 104.29875) (end 174.04375 107.21) (width 0.25) (layer "B.Cu") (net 43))
 (segment (start 143.1925 104.29875) (end 143.1925 109.195) (width 0.25) (layer "B.Cu") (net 37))
 (segment (start 143.1925 109.195) (end 142.36375 110.02375) (width 0.25) (layer "B.Cu") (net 37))
 (segment (start 152.0825 103.384498) (end 152.0825 105.41) (width 0.25) (layer "F.Cu") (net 17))
 (segment (start 145.7325 96.67875) (end 145.7325 98.228002) (width 0.25) (layer "F.Cu") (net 17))
 (segment (start 158.20375 106.45125) (end 157.1625 105.41) (width 0.25) (layer "F.Cu") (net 17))
 (segment (start 149.890501 101.192499) (end 152.0825 103.384498) (width 0.25) (layer "F.Cu") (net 17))
 (segment (start 158.20375 110.02375) (end 158.20375 106.45125) (width 0.25) (layer "F.Cu") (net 17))
 (segment (start 148.696997 101.192499) (end 149.890501 101.192499) (width 0.25) (layer "F.Cu") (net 17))
 (segment (start 145.7325 98.228002) (end 148.696997 101.192499) (width 0.25) (layer "F.Cu") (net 17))
 (via (at 152.0825 105.41) (size 0.8) (drill 0.4) (layers "F.Cu" "B.Cu") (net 17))
 (via (at 157.1625 105.41) (size 0.8) (drill 0.4) (layers "F.Cu" "B.Cu") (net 17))
 (segment (start 156.762501 105.809999) (end 157.1625 105.41) (width 0.25) (layer "B.Cu") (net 17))
 (segment (start 158.20375 106.45125) (end 157.1625 105.41) (width 0.25) (layer "B.Cu") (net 17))
 (segment (start 150.28375 110.02375) (end 150.28375 107.20875) (width 0.25) (layer "B.Cu") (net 17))
 (segment (start 152.482499 105.809999) (end 156.762501 105.809999) (width 0.25) (layer "B.Cu") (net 17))
 (segment (start 158.20375 110.02375) (end 158.20375 106.45125) (width 0.25) (layer "B.Cu") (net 17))
 (segment (start 152.0825 105.41) (end 152.482499 105.809999) (width 0.25) (layer "B.Cu") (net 17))
 (segment (start 150.28375 107.20875) (end 152.0825 105.41) (width 0.25) (layer "B.Cu") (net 17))
 (segment (start 166.0525 109.9525) (end 166.12375 110.02375) (width 0.25) (layer "B.Cu") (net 41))
 (segment (start 166.0525 104.29875) (end 166.0525 109.9525) (width 0.25) (layer "B.Cu") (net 41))
 (segment (start 168.5925 106.045) (end 168.5925 104.29875) (width 0.25) (layer "B.Cu") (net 42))
 (segment (start 170.08375 107.53625) (end 168.5925 106.045) (width 0.25) (layer "B.Cu") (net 42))
 (segment (start 170.08375 110.02375) (end 170.08375 107.53625) (width 0.25) (layer "B.Cu") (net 42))
 (segment (start 175.895 106.52125) (end 173.6725 104.29875) (width 0.25) (layer "B.Cu") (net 44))
 (segment (start 177.00625 106.52125) (end 175.895 106.52125) (width 0.25) (layer "B.Cu") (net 44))
 (segment (start 178.00375 107.51875) (end 177.00625 106.52125) (width 0.25) (layer "B.Cu") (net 44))
 (segment (start 178.00375 110.02375) (end 178.00375 107.51875) (width 0.25) (layer "B.Cu") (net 44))
 (segment (start 154.477501 103.173749) (end 174.452499 103.173749) (width 0.25) (layer "B.Cu") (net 45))
 (segment (start 175.087499 103.808749) (end 175.087499 104.838751) (width 0.25) (layer "B.Cu") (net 45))
 (segment (start 176.319988 106.07124) (end 181.38624 106.07124) (width 0.25) (layer "B.Cu") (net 45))
 (segment (start 153.3525 104.29875) (end 154.477501 103.173749) (width 0.25) (layer "B.Cu") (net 45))
 (segment (start 174.452499 103.173749) (end 175.087499 103.808749) (width 0.25) (layer "B.Cu") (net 45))
 (segment (start 181.38624 106.07124) (end 181.96375 106.64875) (width 0.25) (layer "B.Cu") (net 45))
 (segment (start 181.96375 106.64875) (end 181.96375 110.02375) (width 0.25) (layer "B.Cu") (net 45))
 (segment (start 175.087499 104.838751) (end 176.319988 106.07124) (width 0.25) (layer "B.Cu") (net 45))
 (segment (start 185.92375 108.14875) (end 185.92375 110.02375) (width 0.25) (layer "B.Cu") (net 28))
 (segment (start 180.498739 102.723739) (end 185.92375 108.14875) (width 0.25) (layer "B.Cu") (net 28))
 (segment (start 152.387511 102.723739) (end 180.498739 102.723739) (width 0.25) (layer "B.Cu") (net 28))
 (segment (start 150.8125 104.29875) (end 152.387511 102.723739) (width 0.25) (layer "B.Cu") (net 28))
 (segment (start 182.659238 103.84874) (end 185.92375 107.113252) (width 0.25) (layer "F.Cu") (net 24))
 (segment (start 173.6725 100.093748) (end 177.427492 103.84874) (width 0.25) (layer "F.Cu") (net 24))
 (segment (start 185.92375 107.113252) (end 185.92375 110.02375) (width 0.25) (layer "F.Cu") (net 24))
 (segment (start 173.6725 96.67875) (end 173.6725 100.093748) (width 0.25) (layer "F.Cu") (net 24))
 (segment (start 177.427492 103.84874) (end 182.659238 103.84874) (width 0.25) (layer "F.Cu") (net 24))
 (segment (start 181.96375 110.02375) (end 181.96375 106.64875) (width 0.25) (layer "F.Cu") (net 23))
 (segment (start 181.96375 106.64875) (end 179.61375 104.29875) (width 0.25) (layer "F.Cu") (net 23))
 (segment (start 179.61375 104.29875) (end 176.2125 104.29875) (width 0.25) (layer "F.Cu") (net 23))
 (segment (start 173.8589 105.91249) (end 170.62031 105.91249) (width 0.25) (layer "F.Cu") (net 22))
 (segment (start 174.30891 106.3625) (end 173.8589 105.91249) (width 0.25) (layer "F.Cu") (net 22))
 (segment (start 170.007499 105.299679) (end 170.007499 97.803751) (width 0.25) (layer "F.Cu") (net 22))
 (segment (start 170.62031 105.91249) (end 170.007499 105.299679) (width 0.25) (layer "F.Cu") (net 22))
 (segment (start 178.00375 106.64875) (end 177.7175 106.3625) (width 0.25) (layer "F.Cu") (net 22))
 (segment (start 178.00375 110.02375) (end 178.00375 106.64875) (width 0.25) (layer "F.Cu") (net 22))
 (segment (start 177.7175 106.3625) (end 174.30891 106.3625) (width 0.25) (layer "F.Cu") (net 22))
 (segment (start 170.007499 97.803751) (end 171.1325 96.67875) (width 0.25) (layer "F.Cu") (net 22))
 (segment (start 167.467499 97.803751) (end 168.5925 96.67875) (width 0.25) (layer "F.Cu") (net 21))
 (segment (start 174.04375 106.73375) (end 173.6725 106.3625) (width 0.25) (layer "F.Cu") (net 21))
 (segment (start 174.04375 110.02375) (end 174.04375 106.73375) (width 0.25) (layer "F.Cu") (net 21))
 (segment (start 169.495161 105.423751) (end 168.052499 105.423751) (width 0.25) (layer "F.Cu") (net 21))
 (segment (start 170.43391 106.3625) (end 169.495161 105.423751) (width 0.25) (layer "F.Cu") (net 21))
 (segment (start 167.467499 104.838751) (end 167.467499 97.803751) (width 0.25) (layer "F.Cu") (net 21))
 (segment (start 168.052499 105.423751) (end 167.467499 104.838751) (width 0.25) (layer "F.Cu") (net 21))
 (segment (start 173.6725 106.3625) (end 170.43391 106.3625) (width 0.25) (layer "F.Cu") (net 21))
 (segment (start 166.451248 106.3625) (end 169.7975 106.3625) (width 0.25) (layer "F.Cu") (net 20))
 (segment (start 169.7975 106.3625) (end 170.08375 106.64875) (width 0.25) (layer "F.Cu") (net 20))
 (segment (start 164.927499 104.838751) (end 166.451248 106.3625) (width 0.25) (layer "F.Cu") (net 20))
 (segment (start 170.08375 106.64875) (end 170.08375 110.02375) (width 0.25) (layer "F.Cu") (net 20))
 (segment (start 164.927499 97.803751) (end 164.927499 104.838751) (width 0.25) (layer "F.Cu") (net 20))
 (segment (start 166.0525 96.67875) (end 164.927499 97.803751) (width 0.25) (layer "F.Cu") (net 20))
 (segment (start 162.387499 105.078749) (end 162.387499 97.803751) (width 0.25) (layer "F.Cu") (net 19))
 (segment (start 162.387499 97.803751) (end 163.5125 96.67875) (width 0.25) (layer "F.Cu") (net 19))
 (segment (start 166.12375 107.545) (end 164.94125 106.3625) (width 0.25) (layer "F.Cu") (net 19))
 (segment (start 163.67125 106.3625) (end 162.387499 105.078749) (width 0.25) (layer "F.Cu") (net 19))
 (segment (start 164.94125 106.3625) (end 163.67125 106.3625) (width 0.25) (layer "F.Cu") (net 19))
 (segment (start 166.12375 110.02375) (end 166.12375 107.545) (width 0.25) (layer "F.Cu") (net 19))
 (segment (start 162.16375 108.14875) (end 159.557501 105.542501) (width 0.25) (layer "F.Cu") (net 18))
 (segment (start 158.441253 102.642501) (end 158.084499 102.642501) (width 0.25) (layer "F.Cu") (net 18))
 (segment (start 156.617501 100.261251) (end 154.160001 97.803751) (width 0.25) (layer "F.Cu") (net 18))
 (segment (start 154.160001 97.803751) (end 151.937501 97.803751) (width 0.25) (layer "F.Cu") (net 18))
 (segment (start 156.617501 101.175503) (end 156.617501 100.261251) (width 0.25) (layer "F.Cu") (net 18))
 (segment (start 162.16375 110.02375) (end 162.16375 108.14875) (width 0.25) (layer "F.Cu") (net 18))
 (segment (start 159.557501 105.542501) (end 159.557501 103.758749) (width 0.25) (layer "F.Cu") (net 18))
 (segment (start 151.937501 97.803751) (end 150.8125 96.67875) (width 0.25) (layer "F.Cu") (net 18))
 (segment (start 158.084499 102.642501) (end 156.617501 101.175503) (width 0.25) (layer "F.Cu") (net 18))
 (segment (start 159.557501 103.758749) (end 158.441253 102.642501) (width 0.25) (layer "F.Cu") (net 18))
 (segment (start 154.477501 109.789999) (end 154.24375 110.02375) (width 0.25) (layer "F.Cu") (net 16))
 (segment (start 154.477501 99.708751) (end 154.477501 109.789999) (width 0.25) (layer "F.Cu") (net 16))
 (segment (start 154.46375 99.695) (end 154.477501 99.708751) (width 0.25) (layer "F.Cu") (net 16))
 (segment (start 180.0225 99.695) (end 183.515 103.1875) (width 0.25) (layer "F.Cu") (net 16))
 (segment (start 176.2125 99.695) (end 176.2125 96.67875) (width 0.25) (layer "F.Cu") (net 16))
 (segment (start 176.2125 99.695) (end 180.0225 99.695) (width 0.25) (layer "F.Cu") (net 16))
 (via (at 176.2125 99.695) (size 0.8) (drill 0.4) (layers "F.Cu" "B.Cu") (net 16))
 (via (at 154.46375 99.695) (size 0.8) (drill 0.4) (layers "F.Cu" "B.Cu") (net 16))
 (segment (start 154.46375 99.695) (end 176.2125 99.695) (width 0.25) (layer "B.Cu") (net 16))
 (segment (start 146.32375 106.2475) (end 148.2725 104.29875) (width 0.25) (layer "F.Cu") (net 15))
 (segment (start 146.32375 110.02375) (end 146.32375 106.2475) (width 0.25) (layer "F.Cu") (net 15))
 (segment (start 142.067499 97.803751) (end 142.067499 109.727499) (width 0.25) (layer "F.Cu") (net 14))
 (segment (start 142.067499 109.727499) (end 142.36375 110.02375) (width 0.25) (layer "F.Cu") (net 14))
 (segment (start 143.1925 96.67875) (end 142.067499 97.803751) (width 0.25) (layer "F.Cu") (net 14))
 (segment (start 130.25 105) (end 133 105) (width 0.25) (layer "F.Cu") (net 6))
 (segment (start 116.5 102.75) (end 128 102.75) (width 0.25) (layer "F.Cu") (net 6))
 (segment (start 116 100.5) (end 116 102.25) (width 0.25) (layer "F.Cu") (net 6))
 (segment (start 134.44375 106.44375) (end 134.44375 110.02375) (width 0.25) (layer "F.Cu") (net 6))
 (segment (start 133 105) (end 134.44375 106.44375) (width 0.25) (layer "F.Cu") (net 6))
 (segment (start 128 102.75) (end 130.25 105) (width 0.25) (layer "F.Cu") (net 6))
 (segment (start 116 102.25) (end 116.5 102.75) (width 0.25) (layer "F.Cu") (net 6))
 (segment (start 133 99.25) (end 133 97.65125) (width 0.25) (layer "F.Cu") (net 2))
 (segment (start 133.02 99.27) (end 133.02 102.5525) (width 0.25) (layer "F.Cu") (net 2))
 (segment (start 133 97.65125) (end 133.02 97.63125) (width 0.25) (layer "F.Cu") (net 2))
 (segment (start 148.2725 99.25) (end 148.2725 96.67875) (width 0.25) (layer "F.Cu") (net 2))
 (segment (start 133 99.25) (end 133.02 99.27) (width 0.25) (layer "F.Cu") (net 2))
 (via (at 148.2725 99.25) (size 0.8) (drill 0.4) (layers "F.Cu" "B.Cu") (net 2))
 (via (at 133 99.25) (size 0.8) (drill 0.4) (layers "F.Cu" "B.Cu") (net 2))
 (segment (start 133 99.25) (end 148.2725 99.25) (width 0.25) (layer "B.Cu") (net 2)))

